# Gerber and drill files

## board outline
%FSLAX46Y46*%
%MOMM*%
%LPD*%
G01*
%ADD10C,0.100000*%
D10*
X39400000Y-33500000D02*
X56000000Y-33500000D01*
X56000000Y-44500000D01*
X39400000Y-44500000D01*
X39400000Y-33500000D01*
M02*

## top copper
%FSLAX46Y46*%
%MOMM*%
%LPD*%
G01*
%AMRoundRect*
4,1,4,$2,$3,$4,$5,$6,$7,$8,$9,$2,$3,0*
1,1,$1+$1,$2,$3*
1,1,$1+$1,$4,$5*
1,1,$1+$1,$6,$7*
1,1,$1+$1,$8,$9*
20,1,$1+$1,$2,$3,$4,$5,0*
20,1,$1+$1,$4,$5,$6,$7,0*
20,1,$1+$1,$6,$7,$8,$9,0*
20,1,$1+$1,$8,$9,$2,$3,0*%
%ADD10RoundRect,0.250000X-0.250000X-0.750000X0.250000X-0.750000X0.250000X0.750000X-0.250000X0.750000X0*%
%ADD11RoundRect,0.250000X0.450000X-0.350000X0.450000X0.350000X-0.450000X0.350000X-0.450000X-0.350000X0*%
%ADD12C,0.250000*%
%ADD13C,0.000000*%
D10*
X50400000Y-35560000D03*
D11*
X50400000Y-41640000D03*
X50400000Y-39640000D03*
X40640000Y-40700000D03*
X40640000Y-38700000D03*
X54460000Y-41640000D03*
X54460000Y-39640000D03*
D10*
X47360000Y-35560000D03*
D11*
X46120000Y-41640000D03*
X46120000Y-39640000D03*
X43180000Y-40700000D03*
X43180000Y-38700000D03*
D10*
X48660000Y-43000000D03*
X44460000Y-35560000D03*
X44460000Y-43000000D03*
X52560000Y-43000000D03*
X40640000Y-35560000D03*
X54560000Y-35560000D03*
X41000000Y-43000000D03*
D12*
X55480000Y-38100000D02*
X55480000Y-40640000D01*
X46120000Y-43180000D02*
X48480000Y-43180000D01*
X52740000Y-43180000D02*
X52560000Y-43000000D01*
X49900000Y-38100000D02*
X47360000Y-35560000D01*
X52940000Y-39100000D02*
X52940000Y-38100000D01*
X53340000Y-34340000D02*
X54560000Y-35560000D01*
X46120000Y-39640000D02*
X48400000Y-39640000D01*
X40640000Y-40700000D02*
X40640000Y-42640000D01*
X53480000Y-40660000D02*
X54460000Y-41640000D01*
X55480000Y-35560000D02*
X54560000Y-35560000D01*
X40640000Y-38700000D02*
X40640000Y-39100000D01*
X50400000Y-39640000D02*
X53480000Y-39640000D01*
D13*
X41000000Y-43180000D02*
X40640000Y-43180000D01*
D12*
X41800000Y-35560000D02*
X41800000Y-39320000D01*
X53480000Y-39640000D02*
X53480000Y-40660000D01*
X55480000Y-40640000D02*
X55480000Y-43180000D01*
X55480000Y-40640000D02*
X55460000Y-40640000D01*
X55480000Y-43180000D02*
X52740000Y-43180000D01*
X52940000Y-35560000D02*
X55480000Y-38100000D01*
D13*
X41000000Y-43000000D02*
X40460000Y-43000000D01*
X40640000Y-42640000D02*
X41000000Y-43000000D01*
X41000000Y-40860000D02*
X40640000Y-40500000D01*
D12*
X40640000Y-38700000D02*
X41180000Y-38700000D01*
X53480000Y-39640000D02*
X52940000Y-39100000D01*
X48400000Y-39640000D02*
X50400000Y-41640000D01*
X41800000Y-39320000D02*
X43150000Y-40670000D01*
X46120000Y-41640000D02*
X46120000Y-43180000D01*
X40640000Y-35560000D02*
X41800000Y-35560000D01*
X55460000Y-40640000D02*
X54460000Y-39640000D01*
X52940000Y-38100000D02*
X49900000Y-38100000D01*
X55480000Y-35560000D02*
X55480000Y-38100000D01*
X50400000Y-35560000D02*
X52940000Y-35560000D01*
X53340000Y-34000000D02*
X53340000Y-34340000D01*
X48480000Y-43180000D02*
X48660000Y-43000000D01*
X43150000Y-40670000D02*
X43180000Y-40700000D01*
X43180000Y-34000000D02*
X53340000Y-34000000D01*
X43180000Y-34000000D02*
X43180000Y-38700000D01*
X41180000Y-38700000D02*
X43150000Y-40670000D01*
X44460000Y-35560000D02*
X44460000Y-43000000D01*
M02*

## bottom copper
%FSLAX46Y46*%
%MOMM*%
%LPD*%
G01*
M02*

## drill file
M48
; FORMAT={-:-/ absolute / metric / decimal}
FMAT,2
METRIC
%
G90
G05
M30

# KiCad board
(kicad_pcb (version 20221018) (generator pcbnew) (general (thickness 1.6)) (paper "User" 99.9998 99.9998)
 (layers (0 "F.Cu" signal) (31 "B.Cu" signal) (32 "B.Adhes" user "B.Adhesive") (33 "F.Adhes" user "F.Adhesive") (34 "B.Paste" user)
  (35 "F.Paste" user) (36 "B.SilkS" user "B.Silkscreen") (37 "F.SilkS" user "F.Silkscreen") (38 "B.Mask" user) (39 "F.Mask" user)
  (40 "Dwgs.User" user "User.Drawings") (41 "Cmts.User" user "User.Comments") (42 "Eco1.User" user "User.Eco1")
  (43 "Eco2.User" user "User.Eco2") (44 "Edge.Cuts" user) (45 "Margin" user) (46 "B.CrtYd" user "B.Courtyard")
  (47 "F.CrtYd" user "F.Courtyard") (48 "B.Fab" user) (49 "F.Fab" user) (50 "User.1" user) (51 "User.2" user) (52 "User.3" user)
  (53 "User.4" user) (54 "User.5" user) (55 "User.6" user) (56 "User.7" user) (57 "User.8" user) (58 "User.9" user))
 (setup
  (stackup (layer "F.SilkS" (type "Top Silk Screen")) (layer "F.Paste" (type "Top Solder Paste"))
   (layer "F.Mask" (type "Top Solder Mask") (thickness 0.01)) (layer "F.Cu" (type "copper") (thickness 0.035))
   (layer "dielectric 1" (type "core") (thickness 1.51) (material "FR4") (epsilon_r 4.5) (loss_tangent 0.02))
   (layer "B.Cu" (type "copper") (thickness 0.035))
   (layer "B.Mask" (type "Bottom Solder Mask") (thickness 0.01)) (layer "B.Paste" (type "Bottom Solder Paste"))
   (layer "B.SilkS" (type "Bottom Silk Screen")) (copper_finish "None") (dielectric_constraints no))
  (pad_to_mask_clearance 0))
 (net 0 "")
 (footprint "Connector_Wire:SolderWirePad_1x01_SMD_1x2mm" (layer "F.Cu") (at 50.4 35.56)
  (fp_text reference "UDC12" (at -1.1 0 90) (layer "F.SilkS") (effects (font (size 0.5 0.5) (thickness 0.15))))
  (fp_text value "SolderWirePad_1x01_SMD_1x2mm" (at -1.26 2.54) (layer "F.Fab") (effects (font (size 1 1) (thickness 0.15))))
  (pad "1" smd roundrect (at 0 0) (size 1 2) (layers "F.Cu" "F.Paste" "F.Mask") (roundrect_rratio 0.25)))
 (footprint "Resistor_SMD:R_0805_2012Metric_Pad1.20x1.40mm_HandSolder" (layer "F.Cu") (at 50.4 40.64 90)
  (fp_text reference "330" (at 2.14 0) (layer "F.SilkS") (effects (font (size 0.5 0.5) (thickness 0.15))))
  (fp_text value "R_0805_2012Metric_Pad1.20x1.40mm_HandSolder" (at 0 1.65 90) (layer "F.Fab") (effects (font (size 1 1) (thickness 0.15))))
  (pad "1" smd roundrect (at -1 0 90) (size 1.2 1.4) (layers "F.Cu" "F.Paste" "F.Mask") (roundrect_rratio 0.2083333333))
  (pad "2" smd roundrect (at 1 0 90) (size 1.2 1.4) (layers "F.Cu" "F.Paste" "F.Mask") (roundrect_rratio 0.2083333333)))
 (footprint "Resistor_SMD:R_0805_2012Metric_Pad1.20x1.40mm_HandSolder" (layer "F.Cu") (at 40.64 39.7 90)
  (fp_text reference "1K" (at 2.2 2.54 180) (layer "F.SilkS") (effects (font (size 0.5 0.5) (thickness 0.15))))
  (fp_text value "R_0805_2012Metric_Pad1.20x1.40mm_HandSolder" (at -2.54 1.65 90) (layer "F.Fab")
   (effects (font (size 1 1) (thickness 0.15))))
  (pad "1" smd roundrect (at -1 0 90) (size 1.2 1.4) (layers "F.Cu" "F.Paste" "F.Mask") (roundrect_rratio 0.2083333333))
  (pad "2" smd roundrect (at 1 0 90) (size 1.2 1.4) (layers "F.Cu" "F.Paste" "F.Mask") (roundrect_rratio 0.2083333333)))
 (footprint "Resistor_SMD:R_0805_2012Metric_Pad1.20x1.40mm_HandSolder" (layer "F.Cu") (at 54.46 40.64 90)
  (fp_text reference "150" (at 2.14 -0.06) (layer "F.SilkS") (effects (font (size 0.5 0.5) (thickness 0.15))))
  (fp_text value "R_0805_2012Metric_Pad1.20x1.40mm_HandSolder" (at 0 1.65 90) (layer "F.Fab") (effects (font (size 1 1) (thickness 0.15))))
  (pad "1" smd roundrect (at -1 0 90) (size 1.2 1.4) (layers "F.Cu" "F.Paste" "F.Mask") (roundrect_rratio 0.2083333333))
  (pad "2" smd roundrect (at 1 0 90) (size 1.2 1.4) (layers "F.Cu" "F.Paste" "F.Mask") (roundrect_rratio 0.2083333333)))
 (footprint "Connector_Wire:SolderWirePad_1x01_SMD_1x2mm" (layer "F.Cu") (at 47.36 35.56)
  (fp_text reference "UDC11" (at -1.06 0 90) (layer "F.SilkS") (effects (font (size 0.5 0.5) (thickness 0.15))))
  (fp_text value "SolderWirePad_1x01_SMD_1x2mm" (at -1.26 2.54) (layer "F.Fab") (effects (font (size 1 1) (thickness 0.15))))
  (pad "1" smd roundrect (at 0 0) (size 1 2) (layers "F.Cu" "F.Paste" "F.Mask") (roundrect_rratio 0.25)))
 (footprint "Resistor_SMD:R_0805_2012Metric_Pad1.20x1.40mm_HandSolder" (layer "F.Cu") (at 46.12 40.64 90)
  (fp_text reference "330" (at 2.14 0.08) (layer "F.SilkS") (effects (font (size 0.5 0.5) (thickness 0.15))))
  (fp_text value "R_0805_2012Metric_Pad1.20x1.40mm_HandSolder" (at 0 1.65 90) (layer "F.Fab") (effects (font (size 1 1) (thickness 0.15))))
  (pad "1" smd roundrect (at -1 0 90) (size 1.2 1.4) (layers "F.Cu" "F.Paste" "F.Mask") (roundrect_rratio 0.2083333333))
  (pad "2" smd roundrect (at 1 0 90) (size 1.2 1.4) (layers "F.Cu" "F.Paste" "F.Mask") (roundrect_rratio 0.2083333333)))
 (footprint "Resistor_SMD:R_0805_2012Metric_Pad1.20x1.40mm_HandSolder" (layer "F.Cu") (at 43.18 39.7 90)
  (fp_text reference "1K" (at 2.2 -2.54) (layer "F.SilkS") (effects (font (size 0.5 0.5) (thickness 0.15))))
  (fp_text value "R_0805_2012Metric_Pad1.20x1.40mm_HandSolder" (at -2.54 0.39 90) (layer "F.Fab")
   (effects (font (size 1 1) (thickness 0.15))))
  (pad "1" smd roundrect (at -1 0 90) (size 1.2 1.4) (layers "F.Cu" "F.Paste" "F.Mask") (roundrect_rratio 0.2083333333))
  (pad "2" smd roundrect (at 1 0 90) (size 1.2 1.4) (layers "F.Cu" "F.Paste" "F.Mask") (roundrect_rratio 0.2083333333)))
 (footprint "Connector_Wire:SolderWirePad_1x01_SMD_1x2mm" (layer "F.Cu") (at 48.66 43)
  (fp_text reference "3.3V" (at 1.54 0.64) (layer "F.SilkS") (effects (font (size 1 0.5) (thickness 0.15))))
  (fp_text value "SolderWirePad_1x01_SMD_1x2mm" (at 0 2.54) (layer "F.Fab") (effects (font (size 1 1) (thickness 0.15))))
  (pad "1" smd roundrect (at 0 0) (size 1 2) (layers "F.Cu" "F.Paste" "F.Mask") (roundrect_rratio 0.25)))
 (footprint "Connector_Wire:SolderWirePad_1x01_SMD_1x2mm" (layer "F.Cu") (at 44.46 35.56)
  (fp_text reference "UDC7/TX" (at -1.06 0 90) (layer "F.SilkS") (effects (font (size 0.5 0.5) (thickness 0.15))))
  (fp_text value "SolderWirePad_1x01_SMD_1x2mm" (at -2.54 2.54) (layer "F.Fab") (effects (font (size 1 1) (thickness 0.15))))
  (pad "1" smd roundrect (at 0 0) (size 1 2) (layers "F.Cu" "F.Paste" "F.Mask") (roundrect_rratio 0.25)))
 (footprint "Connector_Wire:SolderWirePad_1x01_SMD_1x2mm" (layer "F.Cu") (at 44.46 43)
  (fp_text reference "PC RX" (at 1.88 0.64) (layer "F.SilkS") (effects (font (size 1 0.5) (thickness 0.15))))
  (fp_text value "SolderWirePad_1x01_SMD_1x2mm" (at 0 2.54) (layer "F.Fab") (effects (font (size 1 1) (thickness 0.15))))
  (pad "1" smd roundrect (at 0 0) (size 1 2) (layers "F.Cu" "F.Paste" "F.Mask") (roundrect_rratio 0.25)))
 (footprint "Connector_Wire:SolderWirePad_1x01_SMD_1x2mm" (layer "F.Cu") (at 52.56 43)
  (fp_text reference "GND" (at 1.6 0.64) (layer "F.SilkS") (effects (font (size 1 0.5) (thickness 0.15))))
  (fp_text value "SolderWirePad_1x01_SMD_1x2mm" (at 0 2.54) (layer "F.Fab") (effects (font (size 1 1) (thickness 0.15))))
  (pad "1" smd roundrect (at 0 0) (size 1 2) (layers "F.Cu" "F.Paste" "F.Mask") (roundrect_rratio 0.25)))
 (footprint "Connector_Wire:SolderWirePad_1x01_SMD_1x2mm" (layer "F.Cu") (at 40.64 35.56)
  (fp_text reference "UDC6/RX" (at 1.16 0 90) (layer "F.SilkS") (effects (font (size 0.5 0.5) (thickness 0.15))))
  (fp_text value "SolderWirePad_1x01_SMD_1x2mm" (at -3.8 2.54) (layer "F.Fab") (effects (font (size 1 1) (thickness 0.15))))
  (pad "1" smd roundrect (at 0 0) (size 1 2) (layers "F.Cu" "F.Paste" "F.Mask") (roundrect_rratio 0.25)))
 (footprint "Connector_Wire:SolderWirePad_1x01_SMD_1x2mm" (layer "F.Cu") (at 54.56 35.56)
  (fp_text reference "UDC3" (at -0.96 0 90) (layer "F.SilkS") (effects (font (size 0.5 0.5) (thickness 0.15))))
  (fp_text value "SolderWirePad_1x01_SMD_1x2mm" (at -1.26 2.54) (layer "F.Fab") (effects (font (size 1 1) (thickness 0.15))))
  (pad "1" smd roundrect (at 0 0) (size 1 2) (layers "F.Cu" "F.Paste" "F.Mask") (roundrect_rratio 0.25)))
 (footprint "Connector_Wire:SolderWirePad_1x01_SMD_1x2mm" (layer "F.Cu") (at 41 43)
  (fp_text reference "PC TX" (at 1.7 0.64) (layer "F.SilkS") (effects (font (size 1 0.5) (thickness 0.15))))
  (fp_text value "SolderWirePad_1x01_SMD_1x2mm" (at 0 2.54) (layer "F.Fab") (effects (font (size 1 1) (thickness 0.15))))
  (pad "1" smd roundrect (at 0 0) (size 1 2) (layers "F.Cu" "F.Paste" "F.Mask") (roundrect_rratio 0.25)))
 (gr_rect (start 39.4 33.5) (end 56 44.5) (stroke (width 0.1) (type default)) (fill none) (layer "Edge.Cuts"))
 (segment (start 55.48 38.1) (end 55.48 40.64) (width 0.25) (layer "F.Cu") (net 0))
 (segment (start 46.12 43.18) (end 48.48 43.18) (width 0.25) (layer "F.Cu") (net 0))
 (segment (start 52.74 43.18) (end 52.56 43) (width 0.25) (layer "F.Cu") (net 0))
 (segment (start 49.9 38.1) (end 47.36 35.56) (width 0.25) (layer "F.Cu") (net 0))
 (segment (start 52.94 39.1) (end 52.94 38.1) (width 0.25) (layer "F.Cu") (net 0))
 (segment (start 53.34 34.34) (end 54.56 35.56) (width 0.25) (layer "F.Cu") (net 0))
 (segment (start 46.12 39.64) (end 48.4 39.64) (width 0.25) (layer "F.Cu") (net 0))
 (segment (start 40.64 40.7) (end 40.64 42.64) (width 0.25) (layer "F.Cu") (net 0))
 (segment (start 53.48 40.66) (end 54.46 41.64) (width 0.25) (layer "F.Cu") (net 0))
 (segment (start 55.48 35.56) (end 54.56 35.56) (width 0.25) (layer "F.Cu") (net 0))
 (segment (start 40.64 38.7) (end 40.64 39.1) (width 0.25) (layer "F.Cu") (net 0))
 (segment (start 50.4 39.64) (end 53.48 39.64) (width 0.25) (layer "F.Cu") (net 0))
 (segment (start 41 43.18) (end 40.64 43.18) (width 0) (layer "F.Cu") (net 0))
 (segment (start 41.8 35.56) (end 41.8 39.32) (width 0.25) (layer "F.Cu") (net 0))
 (segment (start 53.48 39.64) (end 53.48 40.66) (width 0.25) (layer "F.Cu") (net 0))
 (segment (start 55.48 40.64) (end 55.48 43.18) (width 0.25) (layer "F.Cu") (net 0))
 (segment (start 55.48 40.64) (end 55.46 40.64) (width 0.25) (layer "F.Cu") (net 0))
 (segment (start 55.48 43.18) (end 52.74 43.18) (width 0.25) (layer "F.Cu") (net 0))
 (segment (start 52.94 35.56) (end 55.48 38.1) (width 0.25) (layer "F.Cu") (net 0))
 (segment (start 41 43) (end 40.46 43) (width 0) (layer "F.Cu") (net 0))
 (segment (start 40.64 42.64) (end 41 43) (width 0) (layer "F.Cu") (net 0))
 (segment (start 41 40.86) (end 40.64 40.5) (width 0) (layer "F.Cu") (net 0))
 (segment (start 40.64 38.7) (end 41.18 38.7) (width 0.25) (layer "F.Cu") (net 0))
 (segment (start 53.48 39.64) (end 52.94 39.1) (width 0.25) (layer "F.Cu") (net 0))
 (segment (start 48.4 39.64) (end 50.4 41.64) (width 0.25) (layer "F.Cu") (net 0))
 (segment (start 41.8 39.32) (end 43.15 40.67) (width 0.25) (layer "F.Cu") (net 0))
 (segment (start 46.12 41.64) (end 46.12 43.18) (width 0.25) (layer "F.Cu") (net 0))
 (segment (start 40.64 35.56) (end 41.8 35.56) (width 0.25) (layer "F.Cu") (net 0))
 (segment (start 55.46 40.64) (end 54.46 39.64) (width 0.25) (layer "F.Cu") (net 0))
 (segment (start 52.94 38.1) (end 49.9 38.1) (width 0.25) (layer "F.Cu") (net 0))
 (segment (start 55.48 35.56) (end 55.48 38.1) (width 0.25) (layer "F.Cu") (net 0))
 (segment (start 50.4 35.56) (end 52.94 35.56) (width 0.25) (layer "F.Cu") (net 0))
 (segment (start 53.34 34) (end 53.34 34.34) (width 0.25) (layer "F.Cu") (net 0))
 (segment (start 48.48 43.18) (end 48.66 43) (width 0.25) (layer "F.Cu") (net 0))
 (segment (start 43.15 40.67) (end 43.18 40.7) (width 0.25) (layer "F.Cu") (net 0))
 (segment (start 43.18 34) (end 53.34 34) (width 0.25) (layer "F.Cu") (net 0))
 (segment (start 43.18 34) (end 43.18 38.7) (width 0.25) (layer "F.Cu") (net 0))
 (segment (start 41.18 38.7) (end 43.15 40.67) (width 0.25) (layer "F.Cu") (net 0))
 (segment (start 44.46 35.56) (end 44.46 43) (width 0.25) (layer "F.Cu") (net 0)))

